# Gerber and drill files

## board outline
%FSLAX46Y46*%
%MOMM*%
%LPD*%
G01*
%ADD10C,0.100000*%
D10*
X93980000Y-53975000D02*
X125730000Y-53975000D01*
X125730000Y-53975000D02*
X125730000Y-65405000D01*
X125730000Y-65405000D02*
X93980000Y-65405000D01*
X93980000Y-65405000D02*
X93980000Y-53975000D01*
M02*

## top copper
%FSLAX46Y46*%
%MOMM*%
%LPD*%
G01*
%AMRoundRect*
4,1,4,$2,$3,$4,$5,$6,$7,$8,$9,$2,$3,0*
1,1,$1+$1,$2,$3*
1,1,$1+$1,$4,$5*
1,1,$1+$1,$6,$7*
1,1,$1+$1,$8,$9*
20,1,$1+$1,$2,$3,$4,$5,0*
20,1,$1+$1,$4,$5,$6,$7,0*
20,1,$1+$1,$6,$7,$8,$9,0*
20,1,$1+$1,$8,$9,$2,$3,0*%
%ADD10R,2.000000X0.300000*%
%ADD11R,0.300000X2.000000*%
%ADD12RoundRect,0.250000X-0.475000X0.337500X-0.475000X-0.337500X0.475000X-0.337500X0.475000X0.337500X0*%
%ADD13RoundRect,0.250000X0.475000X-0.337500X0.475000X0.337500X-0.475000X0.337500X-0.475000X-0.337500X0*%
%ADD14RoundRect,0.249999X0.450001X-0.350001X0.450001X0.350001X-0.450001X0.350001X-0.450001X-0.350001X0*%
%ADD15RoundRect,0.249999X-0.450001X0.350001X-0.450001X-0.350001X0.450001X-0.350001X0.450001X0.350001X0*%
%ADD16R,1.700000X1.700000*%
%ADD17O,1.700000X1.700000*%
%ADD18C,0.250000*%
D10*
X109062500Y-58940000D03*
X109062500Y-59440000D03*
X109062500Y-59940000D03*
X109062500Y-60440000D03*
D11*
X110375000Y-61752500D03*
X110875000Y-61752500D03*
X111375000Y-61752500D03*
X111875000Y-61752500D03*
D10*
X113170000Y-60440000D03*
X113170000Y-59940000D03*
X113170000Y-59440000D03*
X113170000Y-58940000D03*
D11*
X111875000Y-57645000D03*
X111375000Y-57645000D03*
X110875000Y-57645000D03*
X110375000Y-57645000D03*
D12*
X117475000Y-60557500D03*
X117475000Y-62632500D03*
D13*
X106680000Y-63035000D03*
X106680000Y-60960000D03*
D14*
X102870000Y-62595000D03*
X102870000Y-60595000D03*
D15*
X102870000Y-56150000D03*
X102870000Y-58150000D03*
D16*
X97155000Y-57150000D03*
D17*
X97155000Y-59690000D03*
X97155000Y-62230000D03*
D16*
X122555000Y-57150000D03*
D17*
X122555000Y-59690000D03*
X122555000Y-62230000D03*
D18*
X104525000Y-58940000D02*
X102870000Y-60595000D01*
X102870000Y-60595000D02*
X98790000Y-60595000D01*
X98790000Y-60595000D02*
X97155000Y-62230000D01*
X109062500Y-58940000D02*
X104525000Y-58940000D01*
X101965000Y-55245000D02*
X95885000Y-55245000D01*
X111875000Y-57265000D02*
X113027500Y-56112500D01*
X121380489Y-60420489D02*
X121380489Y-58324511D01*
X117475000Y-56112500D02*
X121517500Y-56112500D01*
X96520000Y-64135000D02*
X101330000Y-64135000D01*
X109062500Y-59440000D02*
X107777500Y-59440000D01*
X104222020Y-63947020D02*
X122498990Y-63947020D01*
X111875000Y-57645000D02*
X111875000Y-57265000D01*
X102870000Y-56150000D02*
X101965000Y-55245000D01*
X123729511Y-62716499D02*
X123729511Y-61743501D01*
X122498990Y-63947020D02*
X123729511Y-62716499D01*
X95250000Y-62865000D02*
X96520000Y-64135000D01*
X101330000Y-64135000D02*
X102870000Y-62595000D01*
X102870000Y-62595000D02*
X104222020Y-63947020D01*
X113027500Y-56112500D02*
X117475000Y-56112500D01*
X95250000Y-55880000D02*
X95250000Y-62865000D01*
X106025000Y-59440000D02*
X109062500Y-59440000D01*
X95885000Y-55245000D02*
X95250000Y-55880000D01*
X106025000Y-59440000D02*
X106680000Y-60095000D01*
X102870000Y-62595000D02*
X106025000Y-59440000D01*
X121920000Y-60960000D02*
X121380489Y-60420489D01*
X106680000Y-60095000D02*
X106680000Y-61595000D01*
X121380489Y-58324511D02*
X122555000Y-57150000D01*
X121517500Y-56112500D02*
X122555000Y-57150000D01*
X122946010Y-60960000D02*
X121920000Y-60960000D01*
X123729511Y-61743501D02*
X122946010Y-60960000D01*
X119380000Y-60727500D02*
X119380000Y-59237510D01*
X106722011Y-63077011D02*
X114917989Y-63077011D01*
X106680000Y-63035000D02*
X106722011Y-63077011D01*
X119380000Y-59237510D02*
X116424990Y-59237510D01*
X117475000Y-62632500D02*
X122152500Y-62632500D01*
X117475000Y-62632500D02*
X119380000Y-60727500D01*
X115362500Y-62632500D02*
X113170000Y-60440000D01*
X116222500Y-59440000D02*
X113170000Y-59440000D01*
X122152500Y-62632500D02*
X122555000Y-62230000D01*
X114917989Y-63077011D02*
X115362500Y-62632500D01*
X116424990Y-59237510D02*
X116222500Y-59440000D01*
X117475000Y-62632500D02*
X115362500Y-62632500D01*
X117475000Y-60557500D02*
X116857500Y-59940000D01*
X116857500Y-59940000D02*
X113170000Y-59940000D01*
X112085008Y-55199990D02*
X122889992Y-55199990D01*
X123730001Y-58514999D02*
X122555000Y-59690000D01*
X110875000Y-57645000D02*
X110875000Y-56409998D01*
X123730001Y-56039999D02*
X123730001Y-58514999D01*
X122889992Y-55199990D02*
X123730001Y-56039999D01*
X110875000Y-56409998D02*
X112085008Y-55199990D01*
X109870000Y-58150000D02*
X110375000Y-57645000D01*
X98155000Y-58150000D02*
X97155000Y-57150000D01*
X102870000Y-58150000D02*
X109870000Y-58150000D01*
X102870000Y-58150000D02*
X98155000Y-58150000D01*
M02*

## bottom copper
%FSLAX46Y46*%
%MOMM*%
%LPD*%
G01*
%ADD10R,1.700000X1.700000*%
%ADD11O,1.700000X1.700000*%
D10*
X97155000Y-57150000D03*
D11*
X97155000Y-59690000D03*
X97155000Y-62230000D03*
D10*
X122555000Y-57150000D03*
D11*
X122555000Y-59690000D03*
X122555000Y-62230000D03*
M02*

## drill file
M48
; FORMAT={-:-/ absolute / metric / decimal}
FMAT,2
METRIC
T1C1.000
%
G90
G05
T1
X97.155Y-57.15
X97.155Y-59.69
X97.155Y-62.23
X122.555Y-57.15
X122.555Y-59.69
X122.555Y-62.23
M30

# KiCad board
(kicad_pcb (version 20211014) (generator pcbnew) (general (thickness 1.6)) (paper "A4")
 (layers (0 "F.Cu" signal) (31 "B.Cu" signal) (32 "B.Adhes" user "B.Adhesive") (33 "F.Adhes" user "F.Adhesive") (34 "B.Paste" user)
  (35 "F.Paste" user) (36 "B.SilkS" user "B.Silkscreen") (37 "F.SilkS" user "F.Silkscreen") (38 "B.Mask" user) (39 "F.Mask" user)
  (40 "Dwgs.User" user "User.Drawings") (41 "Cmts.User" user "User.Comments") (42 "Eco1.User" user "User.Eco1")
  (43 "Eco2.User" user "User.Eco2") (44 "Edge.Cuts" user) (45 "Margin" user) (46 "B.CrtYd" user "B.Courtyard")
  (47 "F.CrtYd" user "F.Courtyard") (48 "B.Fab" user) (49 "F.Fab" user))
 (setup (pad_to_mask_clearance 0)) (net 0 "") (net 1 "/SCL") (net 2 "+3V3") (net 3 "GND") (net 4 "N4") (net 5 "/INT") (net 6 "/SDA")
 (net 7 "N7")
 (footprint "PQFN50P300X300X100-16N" (layer "F.Cu") (at 111.125 59.69)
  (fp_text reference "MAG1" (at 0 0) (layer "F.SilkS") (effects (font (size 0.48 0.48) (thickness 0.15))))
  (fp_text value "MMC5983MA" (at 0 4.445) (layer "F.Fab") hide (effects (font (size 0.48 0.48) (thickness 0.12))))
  (pad "1" smd rect locked (at -2.0625 -0.75) (size 2 0.3) (layers "F.Cu" "F.Paste" "F.Mask") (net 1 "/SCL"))
  (pad "2" smd rect locked (at -2.0625 -0.25) (size 2 0.3) (layers "F.Cu" "F.Paste" "F.Mask") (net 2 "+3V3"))
  (pad "3" smd rect locked (at -2.0625 0.25) (size 2 0.3) (layers "F.Cu" "F.Paste" "F.Mask"))
  (pad "4" smd rect locked (at -2.0625 0.75) (size 2 0.3) (layers "F.Cu" "F.Paste" "F.Mask"))
  (pad "5" smd rect locked (at -0.75 2.0625) (size 0.3 2) (layers "F.Cu" "F.Paste" "F.Mask"))
  (pad "6" smd rect locked (at -0.25 2.0625) (size 0.3 2) (layers "F.Cu" "F.Paste" "F.Mask"))
  (pad "7" smd rect locked (at 0.25 2.0625) (size 0.3 2) (layers "F.Cu" "F.Paste" "F.Mask"))
  (pad "8" smd rect locked (at 0.75 2.0625) (size 0.3 2) (layers "F.Cu" "F.Paste" "F.Mask"))
  (pad "9" smd rect locked (at 2.045 0.75) (size 2 0.3) (layers "F.Cu" "F.Paste" "F.Mask") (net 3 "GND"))
  (pad "10" smd rect locked (at 2.045 0.25) (size 2 0.3) (layers "F.Cu" "F.Paste" "F.Mask") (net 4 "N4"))
  (pad "11" smd rect locked (at 2.045 -0.25) (size 2 0.3) (layers "F.Cu" "F.Paste" "F.Mask") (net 3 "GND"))
  (pad "12" smd rect locked (at 2.045 -0.75) (size 2 0.3) (layers "F.Cu" "F.Paste" "F.Mask"))
  (pad "13" smd rect locked (at 0.75 -2.045) (size 0.3 2) (layers "F.Cu" "F.Paste" "F.Mask") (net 2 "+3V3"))
  (pad "14" smd rect locked (at 0.25 -2.045) (size 0.3 2) (layers "F.Cu" "F.Paste" "F.Mask"))
  (pad "15" smd rect locked (at -0.25 -2.045) (size 0.3 2) (layers "F.Cu" "F.Paste" "F.Mask") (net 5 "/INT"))
  (pad "16" smd rect locked (at -0.75 -2.045) (size 0.3 2) (layers "F.Cu" "F.Paste" "F.Mask") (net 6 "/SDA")))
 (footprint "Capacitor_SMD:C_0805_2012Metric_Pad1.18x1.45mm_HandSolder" (layer "F.Cu") (at 117.475 61.595 -90)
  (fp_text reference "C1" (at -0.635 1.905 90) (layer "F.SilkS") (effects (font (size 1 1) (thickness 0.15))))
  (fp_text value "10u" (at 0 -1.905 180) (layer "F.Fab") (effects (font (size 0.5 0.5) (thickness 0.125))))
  (pad "1" smd roundrect locked (at -1.0375 0 270) (size 1.175 1.45) (layers "F.Cu" "F.Paste" "F.Mask") (roundrect_rratio 0.2127659574)
   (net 4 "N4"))
  (pad "2" smd roundrect locked (at 1.0375 0 270) (size 1.175 1.45) (layers "F.Cu" "F.Paste" "F.Mask") (roundrect_rratio 0.2127659574)
   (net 3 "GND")))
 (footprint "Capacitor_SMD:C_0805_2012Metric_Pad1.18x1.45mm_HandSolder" (layer "F.Cu") (at 106.68 61.9975 90)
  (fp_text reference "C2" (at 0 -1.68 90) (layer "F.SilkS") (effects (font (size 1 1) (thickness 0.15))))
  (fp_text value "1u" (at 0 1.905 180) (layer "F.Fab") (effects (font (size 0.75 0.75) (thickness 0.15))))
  (pad "1" smd roundrect locked (at -1.0375 0 90) (size 1.175 1.45) (layers "F.Cu" "F.Paste" "F.Mask") (roundrect_rratio 0.2127659574)
   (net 3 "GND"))
  (pad "2" smd roundrect locked (at 1.0375 0 90) (size 1.175 1.45) (layers "F.Cu" "F.Paste" "F.Mask") (roundrect_rratio 0.2127659574)
   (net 2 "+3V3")))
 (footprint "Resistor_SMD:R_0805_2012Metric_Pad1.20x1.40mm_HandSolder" (layer "F.Cu") (at 102.87 61.595 90)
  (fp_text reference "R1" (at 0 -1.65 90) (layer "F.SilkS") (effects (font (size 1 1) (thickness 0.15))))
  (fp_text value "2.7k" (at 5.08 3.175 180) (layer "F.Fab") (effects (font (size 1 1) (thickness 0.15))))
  (pad "1" smd roundrect locked (at -1 0 90) (size 1.2 1.4) (layers "F.Cu" "F.Paste" "F.Mask") (roundrect_rratio 0.2083325) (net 2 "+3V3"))
  (pad "2" smd roundrect locked (at 1 0 90) (size 1.2 1.4) (layers "F.Cu" "F.Paste" "F.Mask") (roundrect_rratio 0.2083325) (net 1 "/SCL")))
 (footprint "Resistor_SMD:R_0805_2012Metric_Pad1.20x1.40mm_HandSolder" (layer "F.Cu") (at 102.87 57.15 -90)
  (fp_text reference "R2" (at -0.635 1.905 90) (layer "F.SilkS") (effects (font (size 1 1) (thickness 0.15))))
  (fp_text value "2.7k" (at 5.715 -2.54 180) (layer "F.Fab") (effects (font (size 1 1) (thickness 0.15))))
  (pad "1" smd roundrect locked (at -1 0 270) (size 1.2 1.4) (layers "F.Cu" "F.Paste" "F.Mask") (roundrect_rratio 0.2083325) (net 2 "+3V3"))
  (pad "2" smd roundrect locked (at 1 0 270) (size 1.2 1.4) (layers "F.Cu" "F.Paste" "F.Mask") (roundrect_rratio 0.2083325) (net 6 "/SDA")))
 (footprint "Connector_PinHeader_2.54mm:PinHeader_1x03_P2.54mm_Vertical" (layer "F.Cu") (at 97.155 57.15)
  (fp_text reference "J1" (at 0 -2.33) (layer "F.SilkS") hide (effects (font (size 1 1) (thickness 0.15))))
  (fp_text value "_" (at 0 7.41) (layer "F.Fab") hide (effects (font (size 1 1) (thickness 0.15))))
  (pad "1" thru_hole rect locked (at 0 0) (size 1.7 1.7) (drill 1) (layers *.Cu *.Mask) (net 6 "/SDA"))
  (pad "2" thru_hole oval locked (at 0 2.54) (size 1.7 1.7) (drill 1) (layers *.Cu *.Mask) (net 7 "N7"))
  (pad "3" thru_hole oval locked (at 0 5.08) (size 1.7 1.7) (drill 1) (layers *.Cu *.Mask) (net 1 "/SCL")))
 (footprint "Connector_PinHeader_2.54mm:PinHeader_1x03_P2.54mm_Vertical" (layer "F.Cu") (at 122.555 57.15)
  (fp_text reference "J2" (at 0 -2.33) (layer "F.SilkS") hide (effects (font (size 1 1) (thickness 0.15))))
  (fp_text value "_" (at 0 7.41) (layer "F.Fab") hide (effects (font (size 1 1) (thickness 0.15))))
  (pad "1" thru_hole rect locked (at 0 0) (size 1.7 1.7) (drill 1) (layers *.Cu *.Mask) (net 2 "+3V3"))
  (pad "2" thru_hole oval locked (at 0 2.54) (size 1.7 1.7) (drill 1) (layers *.Cu *.Mask) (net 5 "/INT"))
  (pad "3" thru_hole oval locked (at 0 5.08) (size 1.7 1.7) (drill 1) (layers *.Cu *.Mask) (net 3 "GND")))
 (gr_line (start 93.98 53.975) (end 125.73 53.975) (layer "Edge.Cuts") (width 0.1))
 (gr_line (start 125.73 53.975) (end 125.73 65.405) (layer "Edge.Cuts") (width 0.1))
 (gr_line (start 125.73 65.405) (end 93.98 65.405) (layer "Edge.Cuts") (width 0.1))
 (gr_line (start 93.98 65.405) (end 93.98 53.975) (layer "Edge.Cuts") (width 0.1))
 (segment (start 104.525 58.94) (end 102.87 60.595) (width 0.25) (layer "F.Cu") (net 1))
 (segment (start 102.87 60.595) (end 98.79 60.595) (width 0.25) (layer "F.Cu") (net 1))
 (segment (start 98.79 60.595) (end 97.155 62.23) (width 0.25) (layer "F.Cu") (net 1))
 (segment (start 109.0625 58.94) (end 104.525 58.94) (width 0.25) (layer "F.Cu") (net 1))
 (segment (start 101.965 55.245) (end 95.885 55.245) (width 0.25) (layer "F.Cu") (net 2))
 (segment (start 111.875 57.265) (end 113.0275 56.1125) (width 0.25) (layer "F.Cu") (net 2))
 (segment (start 121.380489 60.420489) (end 121.380489 58.324511) (width 0.25) (layer "F.Cu") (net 2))
 (segment (start 117.475 56.1125) (end 121.5175 56.1125) (width 0.25) (layer "F.Cu") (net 2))
 (segment (start 96.52 64.135) (end 101.33 64.135) (width 0.25) (layer "F.Cu") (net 2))
 (segment (start 109.0625 59.44) (end 107.7775 59.44) (width 0.25) (layer "F.Cu") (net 2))
 (segment (start 104.22202 63.94702) (end 122.49899 63.94702) (width 0.25) (layer "F.Cu") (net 2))
 (segment (start 111.875 57.645) (end 111.875 57.265) (width 0.25) (layer "F.Cu") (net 2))
 (segment (start 102.87 56.15) (end 101.965 55.245) (width 0.25) (layer "F.Cu") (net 2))
 (segment (start 123.729511 62.716499) (end 123.729511 61.743501) (width 0.25) (layer "F.Cu") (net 2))
 (segment (start 122.49899 63.94702) (end 123.729511 62.716499) (width 0.25) (layer "F.Cu") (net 2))
 (segment (start 95.25 62.865) (end 96.52 64.135) (width 0.25) (layer "F.Cu") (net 2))
 (segment (start 101.33 64.135) (end 102.87 62.595) (width 0.25) (layer "F.Cu") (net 2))
 (segment (start 102.87 62.595) (end 104.22202 63.94702) (width 0.25) (layer "F.Cu") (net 2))
 (segment (start 113.0275 56.1125) (end 117.475 56.1125) (width 0.25) (layer "F.Cu") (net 2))
 (segment (start 95.25 55.88) (end 95.25 62.865) (width 0.25) (layer "F.Cu") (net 2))
 (segment (start 106.025 59.44) (end 109.0625 59.44) (width 0.25) (layer "F.Cu") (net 2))
 (segment (start 95.885 55.245) (end 95.25 55.88) (width 0.25) (layer "F.Cu") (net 2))
 (segment (start 106.025 59.44) (end 106.68 60.095) (width 0.25) (layer "F.Cu") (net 2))
 (segment (start 102.87 62.595) (end 106.025 59.44) (width 0.25) (layer "F.Cu") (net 2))
 (segment (start 121.92 60.96) (end 121.380489 60.420489) (width 0.25) (layer "F.Cu") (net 2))
 (segment (start 106.68 60.095) (end 106.68 61.595) (width 0.25) (layer "F.Cu") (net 2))
 (segment (start 121.380489 58.324511) (end 122.555 57.15) (width 0.25) (layer "F.Cu") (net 2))
 (segment (start 121.5175 56.1125) (end 122.555 57.15) (width 0.25) (layer "F.Cu") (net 2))
 (segment (start 122.94601 60.96) (end 121.92 60.96) (width 0.25) (layer "F.Cu") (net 2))
 (segment (start 123.729511 61.743501) (end 122.94601 60.96) (width 0.25) (layer "F.Cu") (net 2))
 (segment (start 119.38 60.7275) (end 119.38 59.23751) (width 0.25) (layer "F.Cu") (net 3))
 (segment (start 106.722011 63.077011) (end 114.917989 63.077011) (width 0.25) (layer "F.Cu") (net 3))
 (segment (start 106.68 63.035) (end 106.722011 63.077011) (width 0.25) (layer "F.Cu") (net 3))
 (segment (start 119.38 59.23751) (end 116.42499 59.23751) (width 0.25) (layer "F.Cu") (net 3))
 (segment (start 117.475 62.6325) (end 122.1525 62.6325) (width 0.25) (layer "F.Cu") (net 3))
 (segment (start 117.475 62.6325) (end 119.38 60.7275) (width 0.25) (layer "F.Cu") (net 3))
 (segment (start 115.3625 62.6325) (end 113.17 60.44) (width 0.25) (layer "F.Cu") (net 3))
 (segment (start 116.2225 59.44) (end 113.17 59.44) (width 0.25) (layer "F.Cu") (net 3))
 (segment (start 122.1525 62.6325) (end 122.555 62.23) (width 0.25) (layer "F.Cu") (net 3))
 (segment (start 114.917989 63.077011) (end 115.3625 62.6325) (width 0.25) (layer "F.Cu") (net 3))
 (segment (start 116.42499 59.23751) (end 116.2225 59.44) (width 0.25) (layer "F.Cu") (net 3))
 (segment (start 117.475 62.6325) (end 115.3625 62.6325) (width 0.25) (layer "F.Cu") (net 3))
 (segment (start 117.475 60.5575) (end 116.8575 59.94) (width 0.25) (layer "F.Cu") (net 4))
 (segment (start 116.8575 59.94) (end 113.17 59.94) (width 0.25) (layer "F.Cu") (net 4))
 (segment (start 112.085008 55.19999) (end 122.889992 55.19999) (width 0.25) (layer "F.Cu") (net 5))
 (segment (start 123.730001 58.514999) (end 122.555 59.69) (width 0.25) (layer "F.Cu") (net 5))
 (segment (start 110.875 57.645) (end 110.875 56.409998) (width 0.25) (layer "F.Cu") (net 5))
 (segment (start 123.730001 56.039999) (end 123.730001 58.514999) (width 0.25) (layer "F.Cu") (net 5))
 (segment (start 122.889992 55.19999) (end 123.730001 56.039999) (width 0.25) (layer "F.Cu") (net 5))
 (segment (start 110.875 56.409998) (end 112.085008 55.19999) (width 0.25) (layer "F.Cu") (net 5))
 (segment (start 109.87 58.15) (end 110.375 57.645) (width 0.25) (layer "F.Cu") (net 6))
 (segment (start 98.155 58.15) (end 97.155 57.15) (width 0.25) (layer "F.Cu") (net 6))
 (segment (start 102.87 58.15) (end 109.87 58.15) (width 0.25) (layer "F.Cu") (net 6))
 (segment (start 102.87 58.15) (end 98.155 58.15) (width 0.25) (layer "F.Cu") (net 6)))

